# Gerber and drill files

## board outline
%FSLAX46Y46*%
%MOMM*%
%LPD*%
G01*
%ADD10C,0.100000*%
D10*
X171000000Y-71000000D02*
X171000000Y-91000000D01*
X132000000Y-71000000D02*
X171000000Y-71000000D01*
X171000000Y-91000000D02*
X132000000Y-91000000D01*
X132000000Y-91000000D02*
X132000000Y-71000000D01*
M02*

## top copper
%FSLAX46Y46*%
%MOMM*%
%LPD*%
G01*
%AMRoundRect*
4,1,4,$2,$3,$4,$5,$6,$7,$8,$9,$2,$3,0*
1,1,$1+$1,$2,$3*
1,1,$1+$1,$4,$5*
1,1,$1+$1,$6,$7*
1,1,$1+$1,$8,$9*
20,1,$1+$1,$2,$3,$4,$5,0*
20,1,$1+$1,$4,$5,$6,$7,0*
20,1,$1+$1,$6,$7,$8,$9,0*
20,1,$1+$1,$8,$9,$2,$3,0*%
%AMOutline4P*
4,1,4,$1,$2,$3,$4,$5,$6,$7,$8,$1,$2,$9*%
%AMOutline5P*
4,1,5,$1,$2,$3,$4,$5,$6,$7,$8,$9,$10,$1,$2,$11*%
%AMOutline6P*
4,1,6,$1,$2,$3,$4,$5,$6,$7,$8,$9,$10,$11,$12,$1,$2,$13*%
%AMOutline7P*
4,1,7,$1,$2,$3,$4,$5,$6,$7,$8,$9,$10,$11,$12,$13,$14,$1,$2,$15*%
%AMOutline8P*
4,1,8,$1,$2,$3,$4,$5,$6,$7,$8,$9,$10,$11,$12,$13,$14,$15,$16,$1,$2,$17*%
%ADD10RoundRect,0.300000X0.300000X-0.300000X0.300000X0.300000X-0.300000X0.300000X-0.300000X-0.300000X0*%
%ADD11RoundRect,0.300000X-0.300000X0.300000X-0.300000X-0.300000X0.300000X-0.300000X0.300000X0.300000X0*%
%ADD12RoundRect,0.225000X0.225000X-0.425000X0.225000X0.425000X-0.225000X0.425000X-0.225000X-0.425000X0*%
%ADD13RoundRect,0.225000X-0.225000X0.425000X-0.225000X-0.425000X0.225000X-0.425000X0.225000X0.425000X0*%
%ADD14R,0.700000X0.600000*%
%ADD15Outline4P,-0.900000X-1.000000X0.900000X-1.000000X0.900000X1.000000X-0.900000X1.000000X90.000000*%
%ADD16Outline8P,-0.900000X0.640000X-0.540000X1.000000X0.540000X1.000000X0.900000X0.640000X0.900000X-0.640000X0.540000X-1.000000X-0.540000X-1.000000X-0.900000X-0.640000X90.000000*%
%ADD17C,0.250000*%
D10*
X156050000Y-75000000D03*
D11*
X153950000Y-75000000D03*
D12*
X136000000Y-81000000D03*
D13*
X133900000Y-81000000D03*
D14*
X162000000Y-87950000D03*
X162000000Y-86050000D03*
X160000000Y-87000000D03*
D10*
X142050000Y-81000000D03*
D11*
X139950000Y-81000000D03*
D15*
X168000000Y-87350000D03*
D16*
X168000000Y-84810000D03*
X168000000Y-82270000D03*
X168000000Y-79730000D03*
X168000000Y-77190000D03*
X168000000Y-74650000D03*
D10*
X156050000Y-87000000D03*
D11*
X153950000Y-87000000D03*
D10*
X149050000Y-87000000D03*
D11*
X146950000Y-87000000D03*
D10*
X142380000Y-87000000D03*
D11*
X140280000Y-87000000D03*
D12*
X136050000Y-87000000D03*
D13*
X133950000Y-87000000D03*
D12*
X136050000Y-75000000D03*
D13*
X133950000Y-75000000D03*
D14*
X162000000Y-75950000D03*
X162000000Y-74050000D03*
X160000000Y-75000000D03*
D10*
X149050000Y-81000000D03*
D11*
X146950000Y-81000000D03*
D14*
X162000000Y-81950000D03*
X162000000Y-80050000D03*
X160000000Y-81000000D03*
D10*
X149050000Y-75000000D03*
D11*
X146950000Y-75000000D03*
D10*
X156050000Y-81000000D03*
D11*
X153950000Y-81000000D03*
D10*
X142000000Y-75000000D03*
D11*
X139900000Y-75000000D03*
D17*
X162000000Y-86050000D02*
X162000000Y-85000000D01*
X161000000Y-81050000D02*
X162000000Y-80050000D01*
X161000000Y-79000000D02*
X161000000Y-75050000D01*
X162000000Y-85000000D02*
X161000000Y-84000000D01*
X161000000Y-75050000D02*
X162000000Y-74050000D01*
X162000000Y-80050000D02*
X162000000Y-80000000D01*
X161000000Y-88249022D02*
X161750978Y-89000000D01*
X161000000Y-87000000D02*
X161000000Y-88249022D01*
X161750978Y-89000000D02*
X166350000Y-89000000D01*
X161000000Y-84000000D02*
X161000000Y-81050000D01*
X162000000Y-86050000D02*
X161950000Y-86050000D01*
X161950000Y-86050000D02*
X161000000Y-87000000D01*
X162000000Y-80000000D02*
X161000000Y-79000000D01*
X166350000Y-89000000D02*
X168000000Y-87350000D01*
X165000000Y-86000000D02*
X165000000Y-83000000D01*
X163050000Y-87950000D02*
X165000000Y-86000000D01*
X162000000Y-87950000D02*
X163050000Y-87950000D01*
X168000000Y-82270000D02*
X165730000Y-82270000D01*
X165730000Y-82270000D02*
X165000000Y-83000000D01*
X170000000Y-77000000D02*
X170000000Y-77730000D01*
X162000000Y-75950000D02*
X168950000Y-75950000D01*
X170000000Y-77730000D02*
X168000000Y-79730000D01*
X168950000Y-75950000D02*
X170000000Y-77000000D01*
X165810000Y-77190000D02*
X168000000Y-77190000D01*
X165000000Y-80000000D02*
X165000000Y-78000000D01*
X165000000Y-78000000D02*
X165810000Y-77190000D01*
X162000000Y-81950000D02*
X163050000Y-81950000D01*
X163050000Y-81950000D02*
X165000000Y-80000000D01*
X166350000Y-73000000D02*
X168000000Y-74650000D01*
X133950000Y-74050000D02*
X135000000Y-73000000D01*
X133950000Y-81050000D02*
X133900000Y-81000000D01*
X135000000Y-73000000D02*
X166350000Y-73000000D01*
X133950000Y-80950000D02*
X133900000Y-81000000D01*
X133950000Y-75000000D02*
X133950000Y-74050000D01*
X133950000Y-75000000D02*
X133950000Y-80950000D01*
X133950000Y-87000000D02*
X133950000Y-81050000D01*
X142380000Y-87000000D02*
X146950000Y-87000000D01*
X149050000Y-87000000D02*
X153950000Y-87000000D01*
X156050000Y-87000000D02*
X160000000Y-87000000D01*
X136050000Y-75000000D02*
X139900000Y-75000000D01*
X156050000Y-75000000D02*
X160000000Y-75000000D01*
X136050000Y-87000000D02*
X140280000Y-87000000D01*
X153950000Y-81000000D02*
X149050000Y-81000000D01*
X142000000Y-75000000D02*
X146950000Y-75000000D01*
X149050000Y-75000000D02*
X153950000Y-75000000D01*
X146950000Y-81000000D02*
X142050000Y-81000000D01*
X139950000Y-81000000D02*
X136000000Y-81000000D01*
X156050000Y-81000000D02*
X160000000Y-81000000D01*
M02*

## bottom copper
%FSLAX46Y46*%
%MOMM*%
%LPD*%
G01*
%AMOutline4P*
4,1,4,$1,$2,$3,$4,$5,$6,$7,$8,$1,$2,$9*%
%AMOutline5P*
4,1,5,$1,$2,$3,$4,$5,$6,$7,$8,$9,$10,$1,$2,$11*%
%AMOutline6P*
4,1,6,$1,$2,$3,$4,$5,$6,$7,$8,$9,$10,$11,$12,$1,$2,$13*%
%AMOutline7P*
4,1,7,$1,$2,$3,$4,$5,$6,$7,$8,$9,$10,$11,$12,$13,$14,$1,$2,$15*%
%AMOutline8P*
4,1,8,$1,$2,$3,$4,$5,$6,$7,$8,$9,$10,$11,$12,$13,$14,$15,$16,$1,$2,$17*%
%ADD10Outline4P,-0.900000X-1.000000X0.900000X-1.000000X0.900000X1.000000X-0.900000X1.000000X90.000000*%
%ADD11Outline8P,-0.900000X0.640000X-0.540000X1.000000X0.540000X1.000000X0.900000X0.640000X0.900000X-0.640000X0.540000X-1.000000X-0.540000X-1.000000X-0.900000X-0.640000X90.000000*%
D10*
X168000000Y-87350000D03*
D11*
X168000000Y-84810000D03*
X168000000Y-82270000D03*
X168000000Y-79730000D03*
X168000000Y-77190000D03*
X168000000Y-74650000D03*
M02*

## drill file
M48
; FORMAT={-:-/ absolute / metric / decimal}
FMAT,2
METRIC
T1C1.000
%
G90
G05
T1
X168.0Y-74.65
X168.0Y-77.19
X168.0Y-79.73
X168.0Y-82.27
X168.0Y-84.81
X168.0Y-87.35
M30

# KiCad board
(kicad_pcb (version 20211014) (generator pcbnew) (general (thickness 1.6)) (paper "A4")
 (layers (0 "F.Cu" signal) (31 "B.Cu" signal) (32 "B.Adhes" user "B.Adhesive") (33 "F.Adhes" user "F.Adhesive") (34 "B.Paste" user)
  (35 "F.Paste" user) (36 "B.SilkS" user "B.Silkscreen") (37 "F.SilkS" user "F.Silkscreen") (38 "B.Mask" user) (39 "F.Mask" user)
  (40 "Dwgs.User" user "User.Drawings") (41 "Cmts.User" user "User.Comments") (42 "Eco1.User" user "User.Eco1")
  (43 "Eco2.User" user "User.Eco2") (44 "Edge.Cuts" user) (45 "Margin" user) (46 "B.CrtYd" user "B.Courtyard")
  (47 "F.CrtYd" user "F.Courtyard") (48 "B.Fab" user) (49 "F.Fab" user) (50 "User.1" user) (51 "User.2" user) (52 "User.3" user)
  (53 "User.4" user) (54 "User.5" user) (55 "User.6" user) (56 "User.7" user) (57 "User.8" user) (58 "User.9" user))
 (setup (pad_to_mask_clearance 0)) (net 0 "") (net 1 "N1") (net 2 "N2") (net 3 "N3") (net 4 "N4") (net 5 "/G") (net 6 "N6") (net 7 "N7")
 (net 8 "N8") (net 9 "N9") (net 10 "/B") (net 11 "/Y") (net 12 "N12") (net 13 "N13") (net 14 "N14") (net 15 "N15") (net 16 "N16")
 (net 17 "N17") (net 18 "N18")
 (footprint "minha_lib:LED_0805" (layer "F.Cu") (at 155 75 180)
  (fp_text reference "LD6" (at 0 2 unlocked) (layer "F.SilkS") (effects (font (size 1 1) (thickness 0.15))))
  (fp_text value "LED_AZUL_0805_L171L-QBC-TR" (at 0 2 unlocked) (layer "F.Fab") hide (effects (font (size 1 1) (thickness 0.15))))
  (pad "1" smd roundrect (at -1.05 0 90) (size 1.2 1.2) (layers "F.Cu" "F.Paste" "F.Mask") (roundrect_rratio 0.25) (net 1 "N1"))
  (pad "2" smd roundrect (at 1.05 0 270) (size 1.2 1.2) (layers "F.Cu" "F.Paste" "F.Mask") (roundrect_rratio 0.25) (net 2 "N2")))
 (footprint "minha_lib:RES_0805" (layer "F.Cu") (at 134.95 81 180)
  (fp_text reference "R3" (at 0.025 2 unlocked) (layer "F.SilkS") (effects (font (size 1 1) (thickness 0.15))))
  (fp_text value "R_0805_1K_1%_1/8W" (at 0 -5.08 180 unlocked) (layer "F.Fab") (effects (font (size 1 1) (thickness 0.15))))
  (pad "1" smd roundrect (at -1.05 0 90) (size 1.3 0.9) (layers "F.Cu" "F.Paste" "F.Mask") (roundrect_rratio 0.25) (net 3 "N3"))
  (pad "2" smd roundrect (at 1.05 0 270) (size 1.3 0.9) (layers "F.Cu" "F.Paste" "F.Mask") (roundrect_rratio 0.25) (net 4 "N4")))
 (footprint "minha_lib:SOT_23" (layer "F.Cu") (at 161 87 -90)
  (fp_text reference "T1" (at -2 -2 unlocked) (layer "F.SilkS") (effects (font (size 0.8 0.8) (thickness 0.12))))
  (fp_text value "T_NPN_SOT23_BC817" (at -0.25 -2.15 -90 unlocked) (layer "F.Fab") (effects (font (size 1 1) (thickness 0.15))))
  (pad "1" smd rect (at 0.95 -1) (size 0.7 0.6) (layers "F.Cu" "F.Paste" "F.Mask") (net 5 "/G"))
  (pad "2" smd rect (at -0.95 -1) (size 0.7 0.6) (layers "F.Cu" "F.Paste" "F.Mask") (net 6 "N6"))
  (pad "3" smd rect (at 0 1 180) (size 0.7 0.6) (layers "F.Cu" "F.Paste" "F.Mask") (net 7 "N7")))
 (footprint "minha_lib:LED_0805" (layer "F.Cu") (at 141 81 180)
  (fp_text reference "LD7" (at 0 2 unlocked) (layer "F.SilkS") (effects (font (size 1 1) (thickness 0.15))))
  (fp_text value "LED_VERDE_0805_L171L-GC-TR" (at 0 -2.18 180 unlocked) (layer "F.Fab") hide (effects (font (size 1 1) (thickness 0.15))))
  (pad "1" smd roundrect (at -1.05 0 90) (size 1.2 1.2) (layers "F.Cu" "F.Paste" "F.Mask") (roundrect_rratio 0.25) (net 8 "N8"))
  (pad "2" smd roundrect (at 1.05 0 270) (size 1.2 1.2) (layers "F.Cu" "F.Paste" "F.Mask") (roundrect_rratio 0.25) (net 3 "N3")))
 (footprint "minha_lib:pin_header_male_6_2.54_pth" (layer "F.Cu") (at 168 87.35 90)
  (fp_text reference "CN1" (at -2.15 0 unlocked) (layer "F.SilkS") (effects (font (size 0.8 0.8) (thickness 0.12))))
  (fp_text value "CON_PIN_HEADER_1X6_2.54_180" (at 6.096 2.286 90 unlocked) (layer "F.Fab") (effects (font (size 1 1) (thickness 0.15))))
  (pad "1" thru_hole trapezoid (at 0 0 90) (size 1.8 2) (drill 1) (layers *.Cu *.Mask) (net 6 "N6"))
  (pad "2" thru_hole roundrect (at 2.54 0 90) (size 1.8 2) (drill 1) (layers *.Cu *.Mask) (roundrect_rratio 0) (chamfer_ratio 0.2)
   (chamfer top_left top_right bottom_left bottom_right) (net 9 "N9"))
  (pad "3" thru_hole roundrect (at 5.08 0 90) (size 1.8 2) (drill 1) (layers *.Cu *.Mask) (roundrect_rratio 0) (chamfer_ratio 0.2)
   (chamfer top_left top_right bottom_left bottom_right) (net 5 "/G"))
  (pad "4" thru_hole roundrect (at 7.62 0 90) (size 1.8 2) (drill 1) (layers *.Cu *.Mask) (roundrect_rratio 0) (chamfer_ratio 0.2)
   (chamfer top_left top_right bottom_left bottom_right) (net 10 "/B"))
  (pad "5" thru_hole roundrect (at 10.16 0 90) (size 1.8 2) (drill 1) (layers *.Cu *.Mask) (roundrect_rratio 0) (chamfer_ratio 0.2)
   (chamfer top_left top_right bottom_left bottom_right) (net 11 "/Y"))
  (pad "6" thru_hole roundrect (at 12.7 0 90) (size 1.8 2) (drill 1) (layers *.Cu *.Mask) (roundrect_rratio 0) (chamfer_ratio 0.2)
   (chamfer top_left top_right bottom_left bottom_right) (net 4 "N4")))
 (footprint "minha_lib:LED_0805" (layer "F.Cu") (at 155 87 180)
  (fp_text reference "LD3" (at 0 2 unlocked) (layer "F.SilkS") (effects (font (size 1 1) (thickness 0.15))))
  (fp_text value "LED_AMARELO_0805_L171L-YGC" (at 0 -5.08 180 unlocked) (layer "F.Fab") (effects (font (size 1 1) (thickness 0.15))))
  (pad "1" smd roundrect (at -1.05 0 90) (size 1.2 1.2) (layers "F.Cu" "F.Paste" "F.Mask") (roundrect_rratio 0.25) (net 7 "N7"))
  (pad "2" smd roundrect (at 1.05 0 270) (size 1.2 1.2) (layers "F.Cu" "F.Paste" "F.Mask") (roundrect_rratio 0.25) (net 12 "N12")))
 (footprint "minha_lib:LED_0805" (layer "F.Cu") (at 148 87 180)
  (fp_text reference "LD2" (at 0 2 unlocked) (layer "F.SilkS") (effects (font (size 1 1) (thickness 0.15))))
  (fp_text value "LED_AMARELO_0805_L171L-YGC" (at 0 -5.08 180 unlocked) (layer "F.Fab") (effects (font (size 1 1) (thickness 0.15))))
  (pad "1" smd roundrect (at -1.05 0 90) (size 1.2 1.2) (layers "F.Cu" "F.Paste" "F.Mask") (roundrect_rratio 0.25) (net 12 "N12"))
  (pad "2" smd roundrect (at 1.05 0 270) (size 1.2 1.2) (layers "F.Cu" "F.Paste" "F.Mask") (roundrect_rratio 0.25) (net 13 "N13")))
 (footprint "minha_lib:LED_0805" (layer "F.Cu") (at 141.33 87 180)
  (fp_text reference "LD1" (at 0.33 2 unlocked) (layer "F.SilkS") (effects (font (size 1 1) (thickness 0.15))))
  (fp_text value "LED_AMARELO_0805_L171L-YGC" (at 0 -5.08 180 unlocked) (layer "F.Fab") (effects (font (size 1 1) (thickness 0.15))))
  (pad "1" smd roundrect (at -1.05 0 90) (size 1.2 1.2) (layers "F.Cu" "F.Paste" "F.Mask") (roundrect_rratio 0.25) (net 13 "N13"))
  (pad "2" smd roundrect (at 1.05 0 270) (size 1.2 1.2) (layers "F.Cu" "F.Paste" "F.Mask") (roundrect_rratio 0.25) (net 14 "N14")))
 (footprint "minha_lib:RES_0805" (layer "F.Cu") (at 135 87 180)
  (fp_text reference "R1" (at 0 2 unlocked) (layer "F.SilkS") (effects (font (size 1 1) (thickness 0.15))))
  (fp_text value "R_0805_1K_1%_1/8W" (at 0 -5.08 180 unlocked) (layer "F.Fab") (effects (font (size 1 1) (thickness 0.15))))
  (pad "1" smd roundrect (at -1.05 0 90) (size 1.3 0.9) (layers "F.Cu" "F.Paste" "F.Mask") (roundrect_rratio 0.25) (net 14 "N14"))
  (pad "2" smd roundrect (at 1.05 0 270) (size 1.3 0.9) (layers "F.Cu" "F.Paste" "F.Mask") (roundrect_rratio 0.25) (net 4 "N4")))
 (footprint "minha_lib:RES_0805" (layer "F.Cu") (at 135 75 180)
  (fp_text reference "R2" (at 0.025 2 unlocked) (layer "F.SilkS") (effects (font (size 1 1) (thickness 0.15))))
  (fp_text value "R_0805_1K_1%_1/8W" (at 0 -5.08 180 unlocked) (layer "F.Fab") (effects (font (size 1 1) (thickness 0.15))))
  (pad "1" smd roundrect (at -1.05 0 90) (size 1.3 0.9) (layers "F.Cu" "F.Paste" "F.Mask") (roundrect_rratio 0.25) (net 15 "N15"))
  (pad "2" smd roundrect (at 1.05 0 270) (size 1.3 0.9) (layers "F.Cu" "F.Paste" "F.Mask") (roundrect_rratio 0.25) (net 4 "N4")))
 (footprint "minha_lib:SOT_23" (layer "F.Cu") (at 161 75 -90)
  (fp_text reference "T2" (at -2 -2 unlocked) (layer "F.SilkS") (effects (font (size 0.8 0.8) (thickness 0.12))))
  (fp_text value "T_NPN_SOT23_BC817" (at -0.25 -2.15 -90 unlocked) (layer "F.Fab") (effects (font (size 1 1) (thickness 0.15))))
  (pad "1" smd rect (at 0.95 -1) (size 0.7 0.6) (layers "F.Cu" "F.Paste" "F.Mask") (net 10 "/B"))
  (pad "2" smd rect (at -0.95 -1) (size 0.7 0.6) (layers "F.Cu" "F.Paste" "F.Mask") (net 6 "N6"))
  (pad "3" smd rect (at 0 1 180) (size 0.7 0.6) (layers "F.Cu" "F.Paste" "F.Mask") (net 1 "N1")))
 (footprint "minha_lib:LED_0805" (layer "F.Cu") (at 148 81 180)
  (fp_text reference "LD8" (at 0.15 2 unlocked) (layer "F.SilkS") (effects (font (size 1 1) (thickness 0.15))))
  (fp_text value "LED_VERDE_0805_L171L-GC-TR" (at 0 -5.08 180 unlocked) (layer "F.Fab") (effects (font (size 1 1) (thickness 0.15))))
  (pad "1" smd roundrect (at -1.05 0 90) (size 1.2 1.2) (layers "F.Cu" "F.Paste" "F.Mask") (roundrect_rratio 0.25) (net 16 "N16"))
  (pad "2" smd roundrect (at 1.05 0 270) (size 1.2 1.2) (layers "F.Cu" "F.Paste" "F.Mask") (roundrect_rratio 0.25) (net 8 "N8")))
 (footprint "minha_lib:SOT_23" (layer "F.Cu") (at 161 81 -90)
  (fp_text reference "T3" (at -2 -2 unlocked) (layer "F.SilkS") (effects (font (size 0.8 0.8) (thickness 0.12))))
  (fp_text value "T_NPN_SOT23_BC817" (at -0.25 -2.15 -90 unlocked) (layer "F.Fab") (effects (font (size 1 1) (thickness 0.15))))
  (pad "1" smd rect (at 0.95 -1) (size 0.7 0.6) (layers "F.Cu" "F.Paste" "F.Mask") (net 11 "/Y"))
  (pad "2" smd rect (at -0.95 -1) (size 0.7 0.6) (layers "F.Cu" "F.Paste" "F.Mask") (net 6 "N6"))
  (pad "3" smd rect (at 0 1 180) (size 0.7 0.6) (layers "F.Cu" "F.Paste" "F.Mask") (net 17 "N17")))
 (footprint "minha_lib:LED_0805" (layer "F.Cu") (at 148 75 180)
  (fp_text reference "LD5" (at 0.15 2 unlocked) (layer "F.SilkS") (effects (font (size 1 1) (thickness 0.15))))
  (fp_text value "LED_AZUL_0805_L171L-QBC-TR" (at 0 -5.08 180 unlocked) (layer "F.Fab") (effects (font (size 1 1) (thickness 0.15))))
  (pad "1" smd roundrect (at -1.05 0 90) (size 1.2 1.2) (layers "F.Cu" "F.Paste" "F.Mask") (roundrect_rratio 0.25) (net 2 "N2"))
  (pad "2" smd roundrect (at 1.05 0 270) (size 1.2 1.2) (layers "F.Cu" "F.Paste" "F.Mask") (roundrect_rratio 0.25) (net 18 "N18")))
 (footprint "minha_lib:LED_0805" (layer "F.Cu") (at 155 81 180)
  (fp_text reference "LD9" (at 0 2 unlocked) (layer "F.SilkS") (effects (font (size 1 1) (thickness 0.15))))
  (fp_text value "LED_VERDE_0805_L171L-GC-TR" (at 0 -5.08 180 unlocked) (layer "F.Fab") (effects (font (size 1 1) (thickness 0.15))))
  (pad "1" smd roundrect (at -1.05 0 90) (size 1.2 1.2) (layers "F.Cu" "F.Paste" "F.Mask") (roundrect_rratio 0.25) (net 17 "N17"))
  (pad "2" smd roundrect (at 1.05 0 270) (size 1.2 1.2) (layers "F.Cu" "F.Paste" "F.Mask") (roundrect_rratio 0.25) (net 16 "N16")))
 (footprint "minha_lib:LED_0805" (layer "F.Cu") (at 140.95 75 180)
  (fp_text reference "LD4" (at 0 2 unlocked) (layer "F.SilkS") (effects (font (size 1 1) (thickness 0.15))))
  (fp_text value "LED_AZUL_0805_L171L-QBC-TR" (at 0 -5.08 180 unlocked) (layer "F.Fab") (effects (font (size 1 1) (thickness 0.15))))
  (pad "1" smd roundrect (at -1.05 0 90) (size 1.2 1.2) (layers "F.Cu" "F.Paste" "F.Mask") (roundrect_rratio 0.25) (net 18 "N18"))
  (pad "2" smd roundrect (at 1.05 0 270) (size 1.2 1.2) (layers "F.Cu" "F.Paste" "F.Mask") (roundrect_rratio 0.25) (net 15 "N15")))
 (gr_line (start 171 71) (end 171 91) (layer "Edge.Cuts") (width 0.1))
 (gr_line (start 132 71) (end 171 71) (layer "Edge.Cuts") (width 0.1))
 (gr_line (start 171 91) (end 132 91) (layer "Edge.Cuts") (width 0.1))
 (gr_line (start 132 91) (end 132 71) (layer "Edge.Cuts") (width 0.1))
 (segment (start 162 86.05) (end 162 85) (width 0.25) (layer "F.Cu") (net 6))
 (segment (start 161 81.05) (end 162 80.05) (width 0.25) (layer "F.Cu") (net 6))
 (segment (start 161 79) (end 161 75.05) (width 0.25) (layer "F.Cu") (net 6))
 (segment (start 162 85) (end 161 84) (width 0.25) (layer "F.Cu") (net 6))
 (segment (start 161 75.05) (end 162 74.05) (width 0.25) (layer "F.Cu") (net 6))
 (segment (start 162 80.05) (end 162 80) (width 0.25) (layer "F.Cu") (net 6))
 (segment (start 161 88.249022) (end 161.750978 89) (width 0.25) (layer "F.Cu") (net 6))
 (segment (start 161 87) (end 161 88.249022) (width 0.25) (layer "F.Cu") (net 6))
 (segment (start 161.750978 89) (end 166.35 89) (width 0.25) (layer "F.Cu") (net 6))
 (segment (start 161 84) (end 161 81.05) (width 0.25) (layer "F.Cu") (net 6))
 (segment (start 162 86.05) (end 161.95 86.05) (width 0.25) (layer "F.Cu") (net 6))
 (segment (start 161.95 86.05) (end 161 87) (width 0.25) (layer "F.Cu") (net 6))
 (segment (start 162 80) (end 161 79) (width 0.25) (layer "F.Cu") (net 6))
 (segment (start 166.35 89) (end 168 87.35) (width 0.25) (layer "F.Cu") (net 6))
 (segment (start 165 86) (end 165 83) (width 0.25) (layer "F.Cu") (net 5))
 (segment (start 163.05 87.95) (end 165 86) (width 0.25) (layer "F.Cu") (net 5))
 (segment (start 162 87.95) (end 163.05 87.95) (width 0.25) (layer "F.Cu") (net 5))
 (segment (start 168 82.27) (end 165.73 82.27) (width 0.25) (layer "F.Cu") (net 5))
 (segment (start 165.73 82.27) (end 165 83) (width 0.25) (layer "F.Cu") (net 5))
 (segment (start 170 77) (end 170 77.73) (width 0.25) (layer "F.Cu") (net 10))
 (segment (start 162 75.95) (end 168.95 75.95) (width 0.25) (layer "F.Cu") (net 10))
 (segment (start 170 77.73) (end 168 79.73) (width 0.25) (layer "F.Cu") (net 10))
 (segment (start 168.95 75.95) (end 170 77) (width 0.25) (layer "F.Cu") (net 10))
 (segment (start 165.81 77.19) (end 168 77.19) (width 0.25) (layer "F.Cu") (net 11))
 (segment (start 165 80) (end 165 78) (width 0.25) (layer "F.Cu") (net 11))
 (segment (start 165 78) (end 165.81 77.19) (width 0.25) (layer "F.Cu") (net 11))
 (segment (start 162 81.95) (end 163.05 81.95) (width 0.25) (layer "F.Cu") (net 11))
 (segment (start 163.05 81.95) (end 165 80) (width 0.25) (layer "F.Cu") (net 11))
 (segment (start 166.35 73) (end 168 74.65) (width 0.25) (layer "F.Cu") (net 4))
 (segment (start 133.95 74.05) (end 135 73) (width 0.25) (layer "F.Cu") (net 4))
 (segment (start 133.95 81.05) (end 133.9 81) (width 0.25) (layer "F.Cu") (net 4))
 (segment (start 135 73) (end 166.35 73) (width 0.25) (layer "F.Cu") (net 4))
 (segment (start 133.95 80.95) (end 133.9 81) (width 0.25) (layer "F.Cu") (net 4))
 (segment (start 133.95 75) (end 133.95 74.05) (width 0.25) (layer "F.Cu") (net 4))
 (segment (start 133.95 75) (end 133.95 80.95) (width 0.25) (layer "F.Cu") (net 4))
 (segment (start 133.95 87) (end 133.95 81.05) (width 0.25) (layer "F.Cu") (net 4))
 (segment (start 142.38 87) (end 146.95 87) (width 0.25) (layer "F.Cu") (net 13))
 (segment (start 149.05 87) (end 153.95 87) (width 0.25) (layer "F.Cu") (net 12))
 (segment (start 156.05 87) (end 160 87) (width 0.25) (layer "F.Cu") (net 7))
 (segment (start 136.05 75) (end 139.9 75) (width 0.25) (layer "F.Cu") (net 15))
 (segment (start 156.05 75) (end 160 75) (width 0.25) (layer "F.Cu") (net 1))
 (segment (start 136.05 87) (end 140.28 87) (width 0.25) (layer "F.Cu") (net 14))
 (segment (start 153.95 81) (end 149.05 81) (width 0.25) (layer "F.Cu") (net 16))
 (segment (start 142 75) (end 146.95 75) (width 0.25) (layer "F.Cu") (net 18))
 (segment (start 149.05 75) (end 153.95 75) (width 0.25) (layer "F.Cu") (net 2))
 (segment (start 146.95 81) (end 142.05 81) (width 0.25) (layer "F.Cu") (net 8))
 (segment (start 139.95 81) (end 136 81) (width 0.25) (layer "F.Cu") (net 3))
 (segment (start 156.05 81) (end 160 81) (width 0.25) (layer "F.Cu") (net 17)))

